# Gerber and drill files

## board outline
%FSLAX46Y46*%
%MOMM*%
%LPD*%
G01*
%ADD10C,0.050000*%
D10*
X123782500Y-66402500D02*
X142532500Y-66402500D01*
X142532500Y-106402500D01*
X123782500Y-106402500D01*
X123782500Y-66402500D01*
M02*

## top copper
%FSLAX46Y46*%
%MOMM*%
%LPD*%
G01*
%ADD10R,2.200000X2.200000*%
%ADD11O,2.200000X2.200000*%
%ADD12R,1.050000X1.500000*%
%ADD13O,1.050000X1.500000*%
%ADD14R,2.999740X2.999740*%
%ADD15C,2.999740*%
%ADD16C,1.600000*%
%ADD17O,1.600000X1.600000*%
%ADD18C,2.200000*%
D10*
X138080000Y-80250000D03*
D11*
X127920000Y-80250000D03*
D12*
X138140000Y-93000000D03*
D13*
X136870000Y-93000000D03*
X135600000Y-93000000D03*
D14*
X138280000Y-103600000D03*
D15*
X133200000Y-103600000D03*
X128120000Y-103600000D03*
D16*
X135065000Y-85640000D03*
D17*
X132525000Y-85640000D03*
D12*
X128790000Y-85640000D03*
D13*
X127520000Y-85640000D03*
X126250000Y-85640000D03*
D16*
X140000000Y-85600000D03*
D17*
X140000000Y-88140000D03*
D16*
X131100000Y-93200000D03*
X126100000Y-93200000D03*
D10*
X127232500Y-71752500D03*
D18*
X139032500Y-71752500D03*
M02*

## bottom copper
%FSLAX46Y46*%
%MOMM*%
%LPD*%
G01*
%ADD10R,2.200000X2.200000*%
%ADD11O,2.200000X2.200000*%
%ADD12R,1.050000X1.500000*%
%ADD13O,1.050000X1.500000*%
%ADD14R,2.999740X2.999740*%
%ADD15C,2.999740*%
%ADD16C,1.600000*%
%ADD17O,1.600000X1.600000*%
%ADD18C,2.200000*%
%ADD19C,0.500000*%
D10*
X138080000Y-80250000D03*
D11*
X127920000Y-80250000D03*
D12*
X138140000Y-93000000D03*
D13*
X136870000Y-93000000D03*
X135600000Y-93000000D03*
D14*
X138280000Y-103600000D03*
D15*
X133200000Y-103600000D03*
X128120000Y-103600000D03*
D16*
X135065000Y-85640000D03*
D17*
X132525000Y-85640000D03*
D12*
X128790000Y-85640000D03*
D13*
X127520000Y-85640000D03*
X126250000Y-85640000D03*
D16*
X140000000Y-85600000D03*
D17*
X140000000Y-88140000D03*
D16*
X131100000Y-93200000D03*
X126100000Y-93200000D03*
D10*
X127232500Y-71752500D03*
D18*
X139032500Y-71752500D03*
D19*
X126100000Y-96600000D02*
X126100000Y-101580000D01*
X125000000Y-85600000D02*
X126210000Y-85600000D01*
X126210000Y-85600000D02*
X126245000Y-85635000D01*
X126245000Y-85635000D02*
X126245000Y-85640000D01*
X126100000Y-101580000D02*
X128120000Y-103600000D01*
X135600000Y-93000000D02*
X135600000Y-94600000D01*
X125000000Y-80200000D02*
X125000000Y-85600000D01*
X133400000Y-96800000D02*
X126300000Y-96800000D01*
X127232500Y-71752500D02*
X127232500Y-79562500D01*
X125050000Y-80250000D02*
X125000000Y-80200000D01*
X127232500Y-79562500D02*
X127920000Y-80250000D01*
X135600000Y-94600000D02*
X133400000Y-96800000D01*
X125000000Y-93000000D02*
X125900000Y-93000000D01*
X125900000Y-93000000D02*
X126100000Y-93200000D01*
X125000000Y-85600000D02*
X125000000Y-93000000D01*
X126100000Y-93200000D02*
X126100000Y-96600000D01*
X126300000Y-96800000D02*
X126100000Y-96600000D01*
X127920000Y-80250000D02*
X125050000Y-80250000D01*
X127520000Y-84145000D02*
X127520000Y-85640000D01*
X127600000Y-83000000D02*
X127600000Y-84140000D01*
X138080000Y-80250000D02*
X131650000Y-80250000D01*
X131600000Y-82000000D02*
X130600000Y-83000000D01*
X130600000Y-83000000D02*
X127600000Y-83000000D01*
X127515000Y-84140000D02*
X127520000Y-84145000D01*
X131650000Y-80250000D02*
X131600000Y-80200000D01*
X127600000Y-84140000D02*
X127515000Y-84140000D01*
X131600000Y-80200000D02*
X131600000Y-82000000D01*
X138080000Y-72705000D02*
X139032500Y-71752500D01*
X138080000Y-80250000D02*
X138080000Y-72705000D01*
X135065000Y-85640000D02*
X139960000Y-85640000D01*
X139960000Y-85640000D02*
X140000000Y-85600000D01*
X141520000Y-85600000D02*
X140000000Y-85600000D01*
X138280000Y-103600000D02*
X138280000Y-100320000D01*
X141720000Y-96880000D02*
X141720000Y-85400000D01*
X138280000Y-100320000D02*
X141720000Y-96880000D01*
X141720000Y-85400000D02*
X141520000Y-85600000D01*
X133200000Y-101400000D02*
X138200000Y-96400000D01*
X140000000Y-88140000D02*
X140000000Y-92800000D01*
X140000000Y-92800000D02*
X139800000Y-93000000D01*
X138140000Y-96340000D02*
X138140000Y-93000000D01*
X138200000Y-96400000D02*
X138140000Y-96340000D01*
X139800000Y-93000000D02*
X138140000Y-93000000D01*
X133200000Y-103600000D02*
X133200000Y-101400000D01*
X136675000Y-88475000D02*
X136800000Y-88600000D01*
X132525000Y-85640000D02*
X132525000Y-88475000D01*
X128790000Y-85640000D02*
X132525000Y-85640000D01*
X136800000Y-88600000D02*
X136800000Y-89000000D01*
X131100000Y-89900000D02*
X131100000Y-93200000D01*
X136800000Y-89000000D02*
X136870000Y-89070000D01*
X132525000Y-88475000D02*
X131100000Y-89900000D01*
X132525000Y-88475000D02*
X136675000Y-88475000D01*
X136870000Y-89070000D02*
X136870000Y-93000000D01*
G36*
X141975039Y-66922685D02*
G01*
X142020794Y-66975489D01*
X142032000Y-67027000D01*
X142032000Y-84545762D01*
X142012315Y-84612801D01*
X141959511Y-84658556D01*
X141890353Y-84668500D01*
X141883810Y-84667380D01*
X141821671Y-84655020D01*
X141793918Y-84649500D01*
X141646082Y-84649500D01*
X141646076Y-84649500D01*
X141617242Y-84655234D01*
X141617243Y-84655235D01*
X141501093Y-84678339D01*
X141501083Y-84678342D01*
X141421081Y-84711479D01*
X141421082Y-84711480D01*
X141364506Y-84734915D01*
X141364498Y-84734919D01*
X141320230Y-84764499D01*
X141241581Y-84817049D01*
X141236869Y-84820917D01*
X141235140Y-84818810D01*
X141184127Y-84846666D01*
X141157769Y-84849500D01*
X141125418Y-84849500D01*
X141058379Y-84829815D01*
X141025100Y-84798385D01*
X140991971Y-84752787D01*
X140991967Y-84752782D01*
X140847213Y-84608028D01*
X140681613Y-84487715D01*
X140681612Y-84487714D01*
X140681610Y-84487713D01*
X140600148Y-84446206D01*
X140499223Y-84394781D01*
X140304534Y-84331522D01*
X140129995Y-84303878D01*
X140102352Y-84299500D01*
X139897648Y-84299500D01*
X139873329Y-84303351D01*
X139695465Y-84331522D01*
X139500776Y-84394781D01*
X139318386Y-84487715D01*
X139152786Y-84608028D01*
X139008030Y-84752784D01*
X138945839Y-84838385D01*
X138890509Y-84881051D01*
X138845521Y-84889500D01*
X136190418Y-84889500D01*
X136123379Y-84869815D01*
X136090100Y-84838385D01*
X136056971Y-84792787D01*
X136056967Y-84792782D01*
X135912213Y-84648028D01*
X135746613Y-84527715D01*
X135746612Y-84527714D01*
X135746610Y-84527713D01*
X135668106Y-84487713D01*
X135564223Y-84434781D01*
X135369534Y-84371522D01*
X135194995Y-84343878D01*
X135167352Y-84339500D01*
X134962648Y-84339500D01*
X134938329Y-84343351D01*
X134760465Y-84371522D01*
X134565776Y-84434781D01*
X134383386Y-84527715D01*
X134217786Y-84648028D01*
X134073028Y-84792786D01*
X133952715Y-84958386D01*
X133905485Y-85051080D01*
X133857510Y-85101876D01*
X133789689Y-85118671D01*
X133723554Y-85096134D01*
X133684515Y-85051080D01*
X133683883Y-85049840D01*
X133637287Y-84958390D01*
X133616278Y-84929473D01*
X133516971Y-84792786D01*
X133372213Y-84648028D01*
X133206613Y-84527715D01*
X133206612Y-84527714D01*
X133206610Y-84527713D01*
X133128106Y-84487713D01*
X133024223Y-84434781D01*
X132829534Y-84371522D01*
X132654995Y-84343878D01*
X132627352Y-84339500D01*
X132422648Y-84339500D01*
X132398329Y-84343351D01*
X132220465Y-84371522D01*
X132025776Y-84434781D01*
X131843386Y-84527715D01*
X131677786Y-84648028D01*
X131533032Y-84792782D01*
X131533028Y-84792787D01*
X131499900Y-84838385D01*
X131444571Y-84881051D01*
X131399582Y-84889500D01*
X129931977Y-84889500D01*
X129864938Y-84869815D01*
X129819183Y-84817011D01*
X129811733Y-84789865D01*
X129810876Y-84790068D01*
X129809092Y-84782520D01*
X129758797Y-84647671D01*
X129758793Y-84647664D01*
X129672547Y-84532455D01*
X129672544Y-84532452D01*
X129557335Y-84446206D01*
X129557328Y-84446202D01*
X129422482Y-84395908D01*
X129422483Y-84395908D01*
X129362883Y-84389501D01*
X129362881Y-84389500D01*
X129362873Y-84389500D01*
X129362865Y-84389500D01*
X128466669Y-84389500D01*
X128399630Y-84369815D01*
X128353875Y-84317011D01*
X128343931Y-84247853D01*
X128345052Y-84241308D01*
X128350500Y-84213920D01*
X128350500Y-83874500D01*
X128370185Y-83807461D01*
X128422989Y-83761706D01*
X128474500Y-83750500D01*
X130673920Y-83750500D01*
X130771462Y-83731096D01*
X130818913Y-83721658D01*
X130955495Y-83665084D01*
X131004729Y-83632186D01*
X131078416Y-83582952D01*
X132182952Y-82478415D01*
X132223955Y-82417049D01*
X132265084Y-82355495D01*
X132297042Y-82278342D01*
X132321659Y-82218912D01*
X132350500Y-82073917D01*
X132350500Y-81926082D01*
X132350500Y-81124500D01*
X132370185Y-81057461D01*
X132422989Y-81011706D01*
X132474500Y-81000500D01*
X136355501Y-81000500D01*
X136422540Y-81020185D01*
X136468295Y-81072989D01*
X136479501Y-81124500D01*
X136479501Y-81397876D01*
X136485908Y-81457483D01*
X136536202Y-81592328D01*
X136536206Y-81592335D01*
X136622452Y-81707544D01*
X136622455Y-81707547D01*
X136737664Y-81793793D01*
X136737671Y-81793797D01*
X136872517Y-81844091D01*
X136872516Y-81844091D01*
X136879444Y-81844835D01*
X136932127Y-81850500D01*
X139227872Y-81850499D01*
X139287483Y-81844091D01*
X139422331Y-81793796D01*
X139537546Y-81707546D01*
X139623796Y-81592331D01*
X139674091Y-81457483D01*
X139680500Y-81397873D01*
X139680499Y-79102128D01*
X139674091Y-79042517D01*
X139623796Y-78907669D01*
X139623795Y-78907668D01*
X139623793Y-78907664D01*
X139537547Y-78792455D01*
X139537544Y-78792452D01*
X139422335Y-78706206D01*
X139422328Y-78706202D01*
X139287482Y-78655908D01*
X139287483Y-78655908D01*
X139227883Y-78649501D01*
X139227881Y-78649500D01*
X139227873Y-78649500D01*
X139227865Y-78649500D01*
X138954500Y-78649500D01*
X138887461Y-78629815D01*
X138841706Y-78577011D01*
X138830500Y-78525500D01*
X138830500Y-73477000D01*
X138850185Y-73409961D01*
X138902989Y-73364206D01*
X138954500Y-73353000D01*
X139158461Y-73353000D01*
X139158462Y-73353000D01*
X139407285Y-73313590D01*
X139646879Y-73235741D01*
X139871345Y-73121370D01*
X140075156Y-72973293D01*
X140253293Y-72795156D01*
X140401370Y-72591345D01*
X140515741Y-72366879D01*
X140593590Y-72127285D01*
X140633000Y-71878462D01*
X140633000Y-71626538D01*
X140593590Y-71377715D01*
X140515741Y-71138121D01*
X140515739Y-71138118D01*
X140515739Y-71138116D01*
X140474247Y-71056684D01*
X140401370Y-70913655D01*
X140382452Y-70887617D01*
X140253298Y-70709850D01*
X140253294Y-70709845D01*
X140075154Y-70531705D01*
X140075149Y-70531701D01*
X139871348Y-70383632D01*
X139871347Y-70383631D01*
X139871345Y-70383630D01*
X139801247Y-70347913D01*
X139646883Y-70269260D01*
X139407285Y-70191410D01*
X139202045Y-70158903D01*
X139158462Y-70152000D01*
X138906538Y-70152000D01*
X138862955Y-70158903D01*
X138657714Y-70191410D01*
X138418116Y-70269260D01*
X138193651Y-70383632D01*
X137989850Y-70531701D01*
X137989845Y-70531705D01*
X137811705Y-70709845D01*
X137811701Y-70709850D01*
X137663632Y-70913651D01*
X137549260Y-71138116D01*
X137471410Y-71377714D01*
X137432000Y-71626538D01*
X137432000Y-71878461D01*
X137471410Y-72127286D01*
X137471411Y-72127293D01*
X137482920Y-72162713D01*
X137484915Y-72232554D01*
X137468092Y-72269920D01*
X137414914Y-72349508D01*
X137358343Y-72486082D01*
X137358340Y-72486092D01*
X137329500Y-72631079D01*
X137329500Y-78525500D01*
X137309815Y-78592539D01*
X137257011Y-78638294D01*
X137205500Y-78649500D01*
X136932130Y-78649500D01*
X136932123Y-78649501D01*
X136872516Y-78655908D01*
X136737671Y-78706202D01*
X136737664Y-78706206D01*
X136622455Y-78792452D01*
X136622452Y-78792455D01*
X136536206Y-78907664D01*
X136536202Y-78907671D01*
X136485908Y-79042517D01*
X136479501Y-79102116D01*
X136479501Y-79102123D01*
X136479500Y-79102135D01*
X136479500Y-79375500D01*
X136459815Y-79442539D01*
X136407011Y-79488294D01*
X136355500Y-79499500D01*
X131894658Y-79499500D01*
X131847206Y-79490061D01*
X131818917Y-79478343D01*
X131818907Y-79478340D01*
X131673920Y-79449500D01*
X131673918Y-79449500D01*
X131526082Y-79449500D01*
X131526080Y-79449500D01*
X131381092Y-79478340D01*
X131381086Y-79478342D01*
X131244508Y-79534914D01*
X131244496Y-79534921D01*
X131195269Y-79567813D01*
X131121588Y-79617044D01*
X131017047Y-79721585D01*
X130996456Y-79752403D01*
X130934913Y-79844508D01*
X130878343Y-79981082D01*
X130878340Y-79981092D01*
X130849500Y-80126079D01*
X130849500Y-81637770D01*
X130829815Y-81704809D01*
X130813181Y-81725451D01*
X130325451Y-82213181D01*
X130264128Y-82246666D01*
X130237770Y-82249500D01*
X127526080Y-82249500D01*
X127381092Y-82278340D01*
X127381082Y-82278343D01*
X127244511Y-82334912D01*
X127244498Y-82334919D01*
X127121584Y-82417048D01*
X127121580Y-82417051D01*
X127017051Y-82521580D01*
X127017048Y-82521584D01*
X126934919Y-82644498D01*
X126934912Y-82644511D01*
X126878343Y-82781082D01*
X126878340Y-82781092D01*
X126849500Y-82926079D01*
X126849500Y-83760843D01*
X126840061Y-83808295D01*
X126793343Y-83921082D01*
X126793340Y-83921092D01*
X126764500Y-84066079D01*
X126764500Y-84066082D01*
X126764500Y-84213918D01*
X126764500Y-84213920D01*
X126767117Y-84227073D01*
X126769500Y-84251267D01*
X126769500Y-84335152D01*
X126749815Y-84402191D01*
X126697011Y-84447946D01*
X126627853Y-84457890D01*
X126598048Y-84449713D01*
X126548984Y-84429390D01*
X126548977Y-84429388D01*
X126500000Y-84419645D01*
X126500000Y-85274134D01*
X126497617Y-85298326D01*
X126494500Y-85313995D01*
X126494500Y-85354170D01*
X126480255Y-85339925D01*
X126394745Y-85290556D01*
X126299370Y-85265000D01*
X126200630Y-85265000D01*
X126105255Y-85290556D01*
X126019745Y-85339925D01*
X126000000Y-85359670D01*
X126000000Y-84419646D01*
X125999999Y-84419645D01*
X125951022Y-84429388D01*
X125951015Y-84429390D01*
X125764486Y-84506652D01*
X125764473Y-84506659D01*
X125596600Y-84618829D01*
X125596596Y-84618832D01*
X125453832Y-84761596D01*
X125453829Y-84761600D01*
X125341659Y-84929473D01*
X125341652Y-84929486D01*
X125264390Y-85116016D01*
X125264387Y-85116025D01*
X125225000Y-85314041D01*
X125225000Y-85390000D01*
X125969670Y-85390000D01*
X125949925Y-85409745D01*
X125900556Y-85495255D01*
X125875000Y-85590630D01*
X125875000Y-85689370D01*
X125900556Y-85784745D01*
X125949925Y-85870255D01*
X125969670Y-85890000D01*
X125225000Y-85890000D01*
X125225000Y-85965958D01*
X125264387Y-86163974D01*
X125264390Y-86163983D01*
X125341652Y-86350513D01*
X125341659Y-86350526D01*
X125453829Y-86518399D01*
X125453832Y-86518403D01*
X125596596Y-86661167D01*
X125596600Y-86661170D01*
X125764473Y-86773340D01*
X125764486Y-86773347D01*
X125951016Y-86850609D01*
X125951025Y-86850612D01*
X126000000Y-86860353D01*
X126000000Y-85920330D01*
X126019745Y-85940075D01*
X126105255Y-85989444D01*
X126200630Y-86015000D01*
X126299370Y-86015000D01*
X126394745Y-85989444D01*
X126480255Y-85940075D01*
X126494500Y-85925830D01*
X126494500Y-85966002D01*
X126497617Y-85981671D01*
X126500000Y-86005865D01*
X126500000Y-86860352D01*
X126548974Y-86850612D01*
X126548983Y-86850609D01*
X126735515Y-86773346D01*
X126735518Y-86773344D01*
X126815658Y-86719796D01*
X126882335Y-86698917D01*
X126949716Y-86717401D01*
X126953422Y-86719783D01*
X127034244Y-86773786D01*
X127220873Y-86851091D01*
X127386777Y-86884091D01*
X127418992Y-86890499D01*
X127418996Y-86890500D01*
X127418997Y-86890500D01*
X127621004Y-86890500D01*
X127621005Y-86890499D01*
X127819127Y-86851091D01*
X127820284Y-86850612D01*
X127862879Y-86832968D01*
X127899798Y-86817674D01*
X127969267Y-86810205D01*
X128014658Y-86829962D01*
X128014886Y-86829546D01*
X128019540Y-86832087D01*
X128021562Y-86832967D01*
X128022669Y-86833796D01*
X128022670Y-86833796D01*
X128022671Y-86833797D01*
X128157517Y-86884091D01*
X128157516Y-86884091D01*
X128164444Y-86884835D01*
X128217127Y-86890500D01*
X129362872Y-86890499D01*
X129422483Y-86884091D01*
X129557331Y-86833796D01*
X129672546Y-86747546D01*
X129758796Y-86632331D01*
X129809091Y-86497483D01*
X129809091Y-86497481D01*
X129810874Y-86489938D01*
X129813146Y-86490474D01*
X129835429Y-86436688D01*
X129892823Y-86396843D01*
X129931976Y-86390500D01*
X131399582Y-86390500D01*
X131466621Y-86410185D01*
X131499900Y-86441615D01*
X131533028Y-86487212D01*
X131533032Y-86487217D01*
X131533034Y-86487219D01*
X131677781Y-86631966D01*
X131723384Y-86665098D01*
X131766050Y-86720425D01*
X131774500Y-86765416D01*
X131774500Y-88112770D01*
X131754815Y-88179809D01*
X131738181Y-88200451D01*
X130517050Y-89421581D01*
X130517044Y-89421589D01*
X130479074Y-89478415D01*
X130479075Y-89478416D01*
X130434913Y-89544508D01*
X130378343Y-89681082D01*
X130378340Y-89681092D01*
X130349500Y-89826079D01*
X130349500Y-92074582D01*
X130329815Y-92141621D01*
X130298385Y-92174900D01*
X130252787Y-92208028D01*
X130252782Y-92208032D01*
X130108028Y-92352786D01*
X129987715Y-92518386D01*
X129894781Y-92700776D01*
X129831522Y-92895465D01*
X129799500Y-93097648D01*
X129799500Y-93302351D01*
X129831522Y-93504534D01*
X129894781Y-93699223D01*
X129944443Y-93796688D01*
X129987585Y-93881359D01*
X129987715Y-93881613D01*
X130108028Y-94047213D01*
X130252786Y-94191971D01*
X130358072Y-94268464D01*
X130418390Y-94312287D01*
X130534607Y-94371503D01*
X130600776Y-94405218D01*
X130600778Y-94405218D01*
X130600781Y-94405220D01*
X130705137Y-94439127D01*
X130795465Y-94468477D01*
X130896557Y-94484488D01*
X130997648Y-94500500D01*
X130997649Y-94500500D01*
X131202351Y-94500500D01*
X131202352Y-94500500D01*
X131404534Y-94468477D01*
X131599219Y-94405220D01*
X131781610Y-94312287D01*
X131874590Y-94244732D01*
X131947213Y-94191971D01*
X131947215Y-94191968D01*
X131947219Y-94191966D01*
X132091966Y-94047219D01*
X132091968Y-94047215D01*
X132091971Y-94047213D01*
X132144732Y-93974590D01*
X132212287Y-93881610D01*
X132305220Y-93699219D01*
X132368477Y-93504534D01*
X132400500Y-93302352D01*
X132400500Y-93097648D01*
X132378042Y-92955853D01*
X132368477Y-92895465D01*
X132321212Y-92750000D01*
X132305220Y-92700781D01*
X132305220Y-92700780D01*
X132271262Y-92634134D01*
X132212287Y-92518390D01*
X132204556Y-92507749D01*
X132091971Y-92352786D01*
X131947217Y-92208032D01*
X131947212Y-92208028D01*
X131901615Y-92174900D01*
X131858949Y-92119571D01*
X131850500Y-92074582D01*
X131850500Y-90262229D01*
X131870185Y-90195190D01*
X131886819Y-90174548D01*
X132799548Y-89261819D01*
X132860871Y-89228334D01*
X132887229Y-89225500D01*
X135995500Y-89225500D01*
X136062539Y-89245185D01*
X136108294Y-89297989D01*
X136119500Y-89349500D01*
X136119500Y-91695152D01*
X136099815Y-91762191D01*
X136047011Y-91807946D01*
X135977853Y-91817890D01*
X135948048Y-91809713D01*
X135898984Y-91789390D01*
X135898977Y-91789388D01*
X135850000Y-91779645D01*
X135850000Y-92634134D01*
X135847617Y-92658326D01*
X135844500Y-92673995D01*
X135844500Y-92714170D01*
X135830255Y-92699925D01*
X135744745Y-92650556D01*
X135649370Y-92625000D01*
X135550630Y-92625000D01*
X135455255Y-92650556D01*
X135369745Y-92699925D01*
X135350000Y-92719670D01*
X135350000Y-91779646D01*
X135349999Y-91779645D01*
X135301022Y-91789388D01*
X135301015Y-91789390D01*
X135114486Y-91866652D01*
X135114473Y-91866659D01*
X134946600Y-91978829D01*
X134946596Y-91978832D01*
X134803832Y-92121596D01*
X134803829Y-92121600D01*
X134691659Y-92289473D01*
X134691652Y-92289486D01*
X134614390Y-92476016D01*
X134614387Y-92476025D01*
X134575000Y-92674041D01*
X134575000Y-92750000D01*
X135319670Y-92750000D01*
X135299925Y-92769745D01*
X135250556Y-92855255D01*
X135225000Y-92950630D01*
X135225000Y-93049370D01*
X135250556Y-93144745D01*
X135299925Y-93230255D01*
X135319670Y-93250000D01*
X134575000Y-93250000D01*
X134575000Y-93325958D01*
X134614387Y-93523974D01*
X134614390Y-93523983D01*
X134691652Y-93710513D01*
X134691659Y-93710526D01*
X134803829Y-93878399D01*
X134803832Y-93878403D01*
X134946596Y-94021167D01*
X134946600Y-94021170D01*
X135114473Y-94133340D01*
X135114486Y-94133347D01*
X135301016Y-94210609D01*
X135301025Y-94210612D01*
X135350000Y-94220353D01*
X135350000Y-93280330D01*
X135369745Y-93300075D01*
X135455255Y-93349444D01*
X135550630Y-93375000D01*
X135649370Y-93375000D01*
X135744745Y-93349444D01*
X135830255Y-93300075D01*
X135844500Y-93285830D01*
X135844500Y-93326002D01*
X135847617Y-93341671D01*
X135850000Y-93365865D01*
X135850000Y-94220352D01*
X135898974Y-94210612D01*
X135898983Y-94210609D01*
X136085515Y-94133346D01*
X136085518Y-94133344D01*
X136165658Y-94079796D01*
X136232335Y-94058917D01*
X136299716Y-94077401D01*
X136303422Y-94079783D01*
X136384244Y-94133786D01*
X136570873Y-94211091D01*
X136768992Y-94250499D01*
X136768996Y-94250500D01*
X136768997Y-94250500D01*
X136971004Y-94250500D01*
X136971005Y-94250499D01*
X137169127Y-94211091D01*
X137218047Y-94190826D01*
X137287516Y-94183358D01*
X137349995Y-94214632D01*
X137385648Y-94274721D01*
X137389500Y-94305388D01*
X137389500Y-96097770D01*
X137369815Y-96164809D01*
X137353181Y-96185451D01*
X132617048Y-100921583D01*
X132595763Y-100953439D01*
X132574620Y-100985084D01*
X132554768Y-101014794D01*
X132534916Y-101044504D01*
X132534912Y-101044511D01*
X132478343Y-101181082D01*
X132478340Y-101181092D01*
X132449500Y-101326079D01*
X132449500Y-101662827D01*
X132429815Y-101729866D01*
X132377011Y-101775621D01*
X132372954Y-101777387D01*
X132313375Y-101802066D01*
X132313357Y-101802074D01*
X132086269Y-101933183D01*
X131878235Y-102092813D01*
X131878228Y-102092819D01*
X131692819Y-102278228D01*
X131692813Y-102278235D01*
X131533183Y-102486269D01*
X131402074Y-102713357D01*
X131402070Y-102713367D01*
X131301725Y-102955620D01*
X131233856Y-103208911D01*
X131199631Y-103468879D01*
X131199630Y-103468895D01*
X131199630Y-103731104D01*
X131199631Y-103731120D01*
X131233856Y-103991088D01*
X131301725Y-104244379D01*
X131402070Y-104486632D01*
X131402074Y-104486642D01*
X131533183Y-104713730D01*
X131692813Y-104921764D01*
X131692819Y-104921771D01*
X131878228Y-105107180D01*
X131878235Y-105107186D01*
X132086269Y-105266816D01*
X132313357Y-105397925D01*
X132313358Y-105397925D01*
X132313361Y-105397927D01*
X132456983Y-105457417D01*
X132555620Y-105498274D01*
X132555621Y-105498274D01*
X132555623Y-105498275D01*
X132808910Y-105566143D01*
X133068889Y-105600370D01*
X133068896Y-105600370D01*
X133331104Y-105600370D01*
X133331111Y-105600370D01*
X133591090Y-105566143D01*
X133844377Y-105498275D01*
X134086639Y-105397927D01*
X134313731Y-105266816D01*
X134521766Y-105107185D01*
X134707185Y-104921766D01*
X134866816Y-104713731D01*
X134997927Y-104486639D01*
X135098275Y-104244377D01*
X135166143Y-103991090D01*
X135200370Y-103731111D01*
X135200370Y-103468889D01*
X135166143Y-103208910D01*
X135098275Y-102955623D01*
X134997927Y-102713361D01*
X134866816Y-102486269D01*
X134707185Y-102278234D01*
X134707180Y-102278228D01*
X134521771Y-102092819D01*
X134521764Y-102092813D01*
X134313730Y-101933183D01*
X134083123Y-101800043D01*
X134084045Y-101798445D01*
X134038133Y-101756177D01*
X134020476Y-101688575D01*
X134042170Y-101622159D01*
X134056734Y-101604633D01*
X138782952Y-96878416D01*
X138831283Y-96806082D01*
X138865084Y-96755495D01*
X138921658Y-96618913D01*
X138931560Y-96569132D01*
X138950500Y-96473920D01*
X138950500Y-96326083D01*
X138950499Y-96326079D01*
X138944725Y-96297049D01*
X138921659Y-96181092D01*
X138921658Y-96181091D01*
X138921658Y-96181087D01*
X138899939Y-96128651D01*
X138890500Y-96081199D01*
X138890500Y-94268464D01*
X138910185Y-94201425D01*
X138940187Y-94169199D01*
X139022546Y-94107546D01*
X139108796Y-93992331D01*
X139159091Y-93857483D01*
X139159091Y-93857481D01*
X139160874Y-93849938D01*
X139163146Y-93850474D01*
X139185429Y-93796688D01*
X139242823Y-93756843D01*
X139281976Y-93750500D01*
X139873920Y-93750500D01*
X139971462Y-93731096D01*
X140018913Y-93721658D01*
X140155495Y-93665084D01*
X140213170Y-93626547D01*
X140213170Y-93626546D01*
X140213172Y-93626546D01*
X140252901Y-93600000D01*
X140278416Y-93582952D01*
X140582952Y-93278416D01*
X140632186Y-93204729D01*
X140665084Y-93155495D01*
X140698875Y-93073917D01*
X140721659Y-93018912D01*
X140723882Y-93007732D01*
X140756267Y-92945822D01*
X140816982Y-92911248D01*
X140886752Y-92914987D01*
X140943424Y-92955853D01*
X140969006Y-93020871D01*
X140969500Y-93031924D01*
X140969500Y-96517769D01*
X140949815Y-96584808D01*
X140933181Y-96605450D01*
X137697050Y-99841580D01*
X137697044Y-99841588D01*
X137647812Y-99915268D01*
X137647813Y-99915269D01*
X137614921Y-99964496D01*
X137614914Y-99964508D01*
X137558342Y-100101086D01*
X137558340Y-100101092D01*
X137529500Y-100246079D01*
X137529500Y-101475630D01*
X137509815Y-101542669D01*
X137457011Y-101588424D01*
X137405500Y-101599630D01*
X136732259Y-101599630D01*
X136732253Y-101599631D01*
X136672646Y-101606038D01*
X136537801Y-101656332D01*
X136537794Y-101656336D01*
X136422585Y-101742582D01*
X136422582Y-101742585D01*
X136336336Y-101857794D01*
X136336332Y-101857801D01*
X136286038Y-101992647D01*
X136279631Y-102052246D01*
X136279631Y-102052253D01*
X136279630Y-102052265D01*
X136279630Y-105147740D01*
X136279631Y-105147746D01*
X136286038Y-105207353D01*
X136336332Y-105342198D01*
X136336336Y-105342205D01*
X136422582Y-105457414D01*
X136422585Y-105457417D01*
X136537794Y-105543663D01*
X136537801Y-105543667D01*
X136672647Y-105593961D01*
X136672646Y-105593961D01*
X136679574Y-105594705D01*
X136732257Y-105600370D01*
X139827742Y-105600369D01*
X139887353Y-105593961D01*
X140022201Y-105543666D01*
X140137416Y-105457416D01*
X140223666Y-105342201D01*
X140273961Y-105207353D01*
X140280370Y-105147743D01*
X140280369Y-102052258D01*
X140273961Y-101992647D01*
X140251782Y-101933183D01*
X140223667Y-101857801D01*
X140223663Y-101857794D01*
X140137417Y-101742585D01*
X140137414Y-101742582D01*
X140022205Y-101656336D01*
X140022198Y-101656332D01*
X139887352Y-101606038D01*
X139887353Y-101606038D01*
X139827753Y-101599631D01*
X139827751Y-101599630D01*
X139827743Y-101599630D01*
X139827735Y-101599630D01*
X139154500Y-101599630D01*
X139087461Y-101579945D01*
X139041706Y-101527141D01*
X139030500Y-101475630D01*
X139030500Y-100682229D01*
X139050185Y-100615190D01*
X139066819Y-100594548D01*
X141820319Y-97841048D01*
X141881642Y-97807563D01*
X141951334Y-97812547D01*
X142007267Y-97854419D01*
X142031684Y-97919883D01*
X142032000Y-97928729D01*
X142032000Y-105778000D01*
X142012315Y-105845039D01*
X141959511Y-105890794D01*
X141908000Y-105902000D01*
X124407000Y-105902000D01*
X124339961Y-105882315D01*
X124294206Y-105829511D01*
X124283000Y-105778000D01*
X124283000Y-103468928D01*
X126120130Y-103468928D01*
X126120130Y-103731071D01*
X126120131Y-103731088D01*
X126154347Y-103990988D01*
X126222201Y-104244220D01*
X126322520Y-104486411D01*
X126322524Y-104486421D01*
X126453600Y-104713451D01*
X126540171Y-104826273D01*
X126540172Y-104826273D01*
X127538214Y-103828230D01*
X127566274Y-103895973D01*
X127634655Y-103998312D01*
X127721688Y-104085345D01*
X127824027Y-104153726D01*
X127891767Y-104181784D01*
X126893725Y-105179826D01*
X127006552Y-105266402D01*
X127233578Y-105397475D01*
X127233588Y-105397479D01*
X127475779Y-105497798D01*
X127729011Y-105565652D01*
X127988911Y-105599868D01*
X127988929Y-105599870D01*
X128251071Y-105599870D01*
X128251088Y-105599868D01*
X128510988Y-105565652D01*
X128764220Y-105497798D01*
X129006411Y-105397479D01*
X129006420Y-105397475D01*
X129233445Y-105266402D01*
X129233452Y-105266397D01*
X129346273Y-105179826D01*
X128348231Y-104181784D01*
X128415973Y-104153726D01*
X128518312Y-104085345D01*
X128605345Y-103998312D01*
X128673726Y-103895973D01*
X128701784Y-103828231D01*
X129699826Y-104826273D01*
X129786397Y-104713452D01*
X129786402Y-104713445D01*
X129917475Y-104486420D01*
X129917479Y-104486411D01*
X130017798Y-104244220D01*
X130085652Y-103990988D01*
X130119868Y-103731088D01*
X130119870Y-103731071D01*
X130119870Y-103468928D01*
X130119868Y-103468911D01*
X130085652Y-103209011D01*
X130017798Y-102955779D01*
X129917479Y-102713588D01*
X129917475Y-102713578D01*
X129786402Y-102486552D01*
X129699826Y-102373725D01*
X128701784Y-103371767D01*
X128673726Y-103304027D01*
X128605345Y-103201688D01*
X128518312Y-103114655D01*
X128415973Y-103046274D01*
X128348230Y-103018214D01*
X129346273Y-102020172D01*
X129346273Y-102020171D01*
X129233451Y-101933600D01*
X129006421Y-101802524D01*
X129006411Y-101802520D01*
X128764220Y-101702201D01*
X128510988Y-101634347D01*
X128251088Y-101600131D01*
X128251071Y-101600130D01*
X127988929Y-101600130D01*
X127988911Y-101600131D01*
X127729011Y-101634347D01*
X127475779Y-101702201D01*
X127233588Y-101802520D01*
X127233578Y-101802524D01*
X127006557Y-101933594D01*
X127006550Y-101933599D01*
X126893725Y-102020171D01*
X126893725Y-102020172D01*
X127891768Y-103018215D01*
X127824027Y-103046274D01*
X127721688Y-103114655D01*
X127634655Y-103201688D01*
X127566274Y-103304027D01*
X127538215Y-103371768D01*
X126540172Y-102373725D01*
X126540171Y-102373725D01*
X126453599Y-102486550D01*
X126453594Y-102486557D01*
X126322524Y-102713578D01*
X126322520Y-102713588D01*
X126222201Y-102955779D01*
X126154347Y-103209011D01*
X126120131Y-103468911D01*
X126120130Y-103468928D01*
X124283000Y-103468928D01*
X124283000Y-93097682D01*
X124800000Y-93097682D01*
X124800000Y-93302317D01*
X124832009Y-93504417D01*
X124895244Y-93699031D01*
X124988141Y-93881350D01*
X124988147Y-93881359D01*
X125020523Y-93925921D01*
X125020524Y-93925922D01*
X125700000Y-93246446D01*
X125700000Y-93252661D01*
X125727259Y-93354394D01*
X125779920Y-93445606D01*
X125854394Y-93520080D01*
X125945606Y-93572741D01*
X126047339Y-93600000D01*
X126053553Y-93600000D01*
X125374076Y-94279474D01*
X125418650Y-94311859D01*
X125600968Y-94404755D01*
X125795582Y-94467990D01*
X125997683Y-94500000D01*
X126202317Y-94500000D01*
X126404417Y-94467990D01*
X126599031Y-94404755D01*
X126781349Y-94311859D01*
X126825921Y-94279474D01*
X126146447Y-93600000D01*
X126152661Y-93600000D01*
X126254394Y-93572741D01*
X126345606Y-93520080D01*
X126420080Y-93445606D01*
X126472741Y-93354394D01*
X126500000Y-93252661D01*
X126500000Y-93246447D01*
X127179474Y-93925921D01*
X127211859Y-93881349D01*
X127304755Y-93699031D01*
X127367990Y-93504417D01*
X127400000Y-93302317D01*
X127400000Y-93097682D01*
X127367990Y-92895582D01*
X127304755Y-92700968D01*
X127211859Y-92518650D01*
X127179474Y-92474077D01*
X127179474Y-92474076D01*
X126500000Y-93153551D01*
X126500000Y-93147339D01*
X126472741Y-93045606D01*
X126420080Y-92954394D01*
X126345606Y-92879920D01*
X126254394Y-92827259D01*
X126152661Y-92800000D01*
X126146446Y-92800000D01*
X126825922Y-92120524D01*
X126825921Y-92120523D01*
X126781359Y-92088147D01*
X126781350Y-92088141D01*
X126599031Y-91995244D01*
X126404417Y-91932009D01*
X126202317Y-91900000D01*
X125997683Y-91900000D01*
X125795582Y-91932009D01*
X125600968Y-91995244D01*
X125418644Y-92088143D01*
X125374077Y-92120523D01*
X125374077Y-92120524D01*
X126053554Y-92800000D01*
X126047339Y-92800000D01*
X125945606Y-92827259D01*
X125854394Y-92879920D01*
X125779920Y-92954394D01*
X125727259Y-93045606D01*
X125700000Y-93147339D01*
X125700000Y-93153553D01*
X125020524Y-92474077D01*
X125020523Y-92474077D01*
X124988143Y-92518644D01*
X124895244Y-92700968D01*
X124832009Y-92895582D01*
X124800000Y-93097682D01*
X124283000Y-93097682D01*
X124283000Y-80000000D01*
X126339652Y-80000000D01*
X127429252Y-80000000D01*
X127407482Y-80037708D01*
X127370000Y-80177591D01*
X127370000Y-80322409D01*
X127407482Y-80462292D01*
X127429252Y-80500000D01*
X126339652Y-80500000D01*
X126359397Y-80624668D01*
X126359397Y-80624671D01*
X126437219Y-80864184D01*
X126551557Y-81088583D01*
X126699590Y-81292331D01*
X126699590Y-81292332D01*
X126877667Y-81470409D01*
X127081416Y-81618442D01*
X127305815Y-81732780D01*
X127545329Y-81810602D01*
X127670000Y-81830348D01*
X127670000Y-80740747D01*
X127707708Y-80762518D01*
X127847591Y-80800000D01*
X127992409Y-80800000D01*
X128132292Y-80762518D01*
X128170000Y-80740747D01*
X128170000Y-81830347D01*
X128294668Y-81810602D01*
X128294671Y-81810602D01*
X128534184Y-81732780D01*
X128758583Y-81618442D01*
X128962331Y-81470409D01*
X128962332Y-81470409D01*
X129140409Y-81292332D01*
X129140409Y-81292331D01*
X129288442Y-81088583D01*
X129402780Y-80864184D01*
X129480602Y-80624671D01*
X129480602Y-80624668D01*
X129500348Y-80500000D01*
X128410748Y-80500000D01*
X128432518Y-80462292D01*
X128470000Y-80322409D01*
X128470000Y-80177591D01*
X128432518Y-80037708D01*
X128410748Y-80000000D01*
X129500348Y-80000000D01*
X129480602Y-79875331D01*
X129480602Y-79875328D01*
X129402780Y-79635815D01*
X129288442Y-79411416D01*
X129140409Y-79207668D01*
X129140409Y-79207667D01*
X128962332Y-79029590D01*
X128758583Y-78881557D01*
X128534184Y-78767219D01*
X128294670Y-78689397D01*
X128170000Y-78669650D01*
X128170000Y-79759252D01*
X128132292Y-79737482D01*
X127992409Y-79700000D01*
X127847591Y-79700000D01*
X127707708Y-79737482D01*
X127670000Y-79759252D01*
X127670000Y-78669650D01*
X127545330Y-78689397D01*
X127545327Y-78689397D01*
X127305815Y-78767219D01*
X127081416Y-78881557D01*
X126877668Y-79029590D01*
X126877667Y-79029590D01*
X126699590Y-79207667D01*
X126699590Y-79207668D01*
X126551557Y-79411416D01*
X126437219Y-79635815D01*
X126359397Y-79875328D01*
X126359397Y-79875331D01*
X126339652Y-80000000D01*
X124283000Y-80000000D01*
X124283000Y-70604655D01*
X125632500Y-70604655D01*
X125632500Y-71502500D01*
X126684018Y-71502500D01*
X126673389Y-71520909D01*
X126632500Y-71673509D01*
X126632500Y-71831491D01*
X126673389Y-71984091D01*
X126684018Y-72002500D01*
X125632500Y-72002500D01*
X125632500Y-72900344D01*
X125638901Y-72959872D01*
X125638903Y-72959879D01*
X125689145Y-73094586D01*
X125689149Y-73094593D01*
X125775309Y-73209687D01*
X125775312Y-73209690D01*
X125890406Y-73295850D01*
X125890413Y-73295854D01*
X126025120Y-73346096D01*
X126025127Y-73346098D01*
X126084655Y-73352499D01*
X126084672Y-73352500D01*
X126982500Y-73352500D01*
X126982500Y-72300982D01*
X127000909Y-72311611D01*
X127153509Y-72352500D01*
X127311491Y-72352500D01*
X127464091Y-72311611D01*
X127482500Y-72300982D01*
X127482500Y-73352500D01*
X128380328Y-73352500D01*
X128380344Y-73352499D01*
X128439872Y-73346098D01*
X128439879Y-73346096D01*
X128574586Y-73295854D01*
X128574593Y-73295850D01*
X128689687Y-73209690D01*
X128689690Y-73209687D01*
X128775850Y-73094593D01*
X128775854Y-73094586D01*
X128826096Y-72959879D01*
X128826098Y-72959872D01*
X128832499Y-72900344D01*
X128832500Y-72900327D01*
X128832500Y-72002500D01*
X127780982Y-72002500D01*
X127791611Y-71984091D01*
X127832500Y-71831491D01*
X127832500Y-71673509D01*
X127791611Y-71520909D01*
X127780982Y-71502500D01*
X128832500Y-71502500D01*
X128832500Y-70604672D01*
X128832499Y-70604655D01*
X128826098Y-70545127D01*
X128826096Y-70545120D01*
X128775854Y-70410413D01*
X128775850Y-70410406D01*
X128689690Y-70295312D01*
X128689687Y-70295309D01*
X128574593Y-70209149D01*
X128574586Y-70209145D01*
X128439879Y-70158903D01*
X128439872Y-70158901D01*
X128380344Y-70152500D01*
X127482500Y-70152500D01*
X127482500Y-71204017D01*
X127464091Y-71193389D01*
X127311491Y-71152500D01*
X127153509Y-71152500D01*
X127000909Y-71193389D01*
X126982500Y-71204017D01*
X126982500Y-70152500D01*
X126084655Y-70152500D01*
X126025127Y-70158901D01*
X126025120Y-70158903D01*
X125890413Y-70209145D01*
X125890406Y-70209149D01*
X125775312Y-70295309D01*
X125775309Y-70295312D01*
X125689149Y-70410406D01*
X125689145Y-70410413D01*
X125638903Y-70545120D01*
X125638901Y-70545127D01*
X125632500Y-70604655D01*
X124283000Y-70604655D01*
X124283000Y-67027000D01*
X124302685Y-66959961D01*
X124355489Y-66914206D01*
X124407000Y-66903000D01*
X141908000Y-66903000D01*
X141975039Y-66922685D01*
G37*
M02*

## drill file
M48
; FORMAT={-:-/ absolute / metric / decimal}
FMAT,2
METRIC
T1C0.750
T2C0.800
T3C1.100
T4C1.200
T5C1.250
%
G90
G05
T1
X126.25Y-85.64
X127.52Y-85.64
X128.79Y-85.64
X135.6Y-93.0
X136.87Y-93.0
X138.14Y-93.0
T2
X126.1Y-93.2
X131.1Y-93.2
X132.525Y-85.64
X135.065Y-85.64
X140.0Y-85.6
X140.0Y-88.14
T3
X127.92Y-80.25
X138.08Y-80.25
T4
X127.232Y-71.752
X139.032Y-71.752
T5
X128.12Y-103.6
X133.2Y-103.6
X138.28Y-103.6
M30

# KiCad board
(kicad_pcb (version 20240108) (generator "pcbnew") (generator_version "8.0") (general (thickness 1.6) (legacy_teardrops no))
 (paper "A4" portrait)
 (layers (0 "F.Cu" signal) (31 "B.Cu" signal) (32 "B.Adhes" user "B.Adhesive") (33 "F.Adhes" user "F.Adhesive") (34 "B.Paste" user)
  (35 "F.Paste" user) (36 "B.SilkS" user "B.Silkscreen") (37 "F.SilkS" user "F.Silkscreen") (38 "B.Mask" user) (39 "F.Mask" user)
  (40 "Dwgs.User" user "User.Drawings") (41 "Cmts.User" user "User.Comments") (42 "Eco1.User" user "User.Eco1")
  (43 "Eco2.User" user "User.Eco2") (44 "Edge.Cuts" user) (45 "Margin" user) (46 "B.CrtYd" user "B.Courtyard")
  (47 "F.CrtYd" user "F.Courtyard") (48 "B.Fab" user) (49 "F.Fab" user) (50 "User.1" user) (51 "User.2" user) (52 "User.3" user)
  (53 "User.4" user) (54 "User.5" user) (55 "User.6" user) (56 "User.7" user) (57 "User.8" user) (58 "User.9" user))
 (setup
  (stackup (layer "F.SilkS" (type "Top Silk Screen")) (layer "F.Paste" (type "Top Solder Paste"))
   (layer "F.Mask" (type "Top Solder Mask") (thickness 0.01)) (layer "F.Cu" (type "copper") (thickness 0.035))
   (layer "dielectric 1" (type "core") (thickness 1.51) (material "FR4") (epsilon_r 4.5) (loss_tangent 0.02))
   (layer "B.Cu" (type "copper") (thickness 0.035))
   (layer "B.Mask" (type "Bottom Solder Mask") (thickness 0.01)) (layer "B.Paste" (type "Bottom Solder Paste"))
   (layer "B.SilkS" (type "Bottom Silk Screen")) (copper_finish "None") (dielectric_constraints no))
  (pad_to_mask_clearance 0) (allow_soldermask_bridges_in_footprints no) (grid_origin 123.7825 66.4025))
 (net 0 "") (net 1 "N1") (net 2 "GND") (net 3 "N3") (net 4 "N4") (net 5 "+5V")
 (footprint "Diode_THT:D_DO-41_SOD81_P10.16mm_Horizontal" (layer "F.Cu") (at 138.08 80.25 180)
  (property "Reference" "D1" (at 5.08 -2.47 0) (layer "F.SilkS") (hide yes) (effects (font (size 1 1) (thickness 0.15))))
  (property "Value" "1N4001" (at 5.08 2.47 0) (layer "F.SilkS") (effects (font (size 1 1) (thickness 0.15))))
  (pad "1" thru_hole rect (at 0 0 180) (size 2.2 2.2) (drill 1.1) (layers "*.Cu" "*.Mask") (remove_unused_layers no) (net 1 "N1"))
  (pad "2" thru_hole oval (at 10.16 0 180) (size 2.2 2.2) (drill 1.1) (layers "*.Cu" "*.Mask") (remove_unused_layers no) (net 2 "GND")))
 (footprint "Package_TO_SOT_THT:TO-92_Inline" (layer "F.Cu") (at 138.14 93 180)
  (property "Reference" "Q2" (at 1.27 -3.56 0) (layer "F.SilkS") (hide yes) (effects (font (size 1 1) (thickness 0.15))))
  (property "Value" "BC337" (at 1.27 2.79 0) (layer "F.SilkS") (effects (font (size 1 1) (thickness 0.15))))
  (pad "1" thru_hole rect (at 0 0 180) (size 1.05 1.5) (drill 0.75) (layers "*.Cu" "*.Mask") (remove_unused_layers no) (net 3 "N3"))
  (pad "2" thru_hole oval (at 1.27 0 180) (size 1.05 1.5) (drill 0.75) (layers "*.Cu" "*.Mask") (remove_unused_layers no) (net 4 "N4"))
  (pad "3" thru_hole oval (at 2.54 0 180) (size 1.05 1.5) (drill 0.75) (layers "*.Cu" "*.Mask") (remove_unused_layers no) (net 2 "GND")))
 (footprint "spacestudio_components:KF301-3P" (layer "F.Cu") (at 133.2 103.6 180)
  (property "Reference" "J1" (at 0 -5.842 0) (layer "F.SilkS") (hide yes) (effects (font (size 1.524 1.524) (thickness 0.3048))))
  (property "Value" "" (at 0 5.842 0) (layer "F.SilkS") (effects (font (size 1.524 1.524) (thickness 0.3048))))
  (pad "1" thru_hole rect (at -5.08 0 180) (size 2.99974 2.99974) (drill 1.24968) (layers "*.Cu" "*.Mask" "F.SilkS")
   (remove_unused_layers no) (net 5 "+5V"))
  (pad "2" thru_hole circle (at 0 0 180) (size 2.99974 2.99974) (drill 1.24968) (layers "*.Cu" "*.Mask" "F.SilkS") (remove_unused_layers no)
   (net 3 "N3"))
  (pad "3" thru_hole circle (at 5.08 0 180) (size 2.99974 2.99974) (drill 1.24968) (layers "*.Cu" "*.Mask" "F.SilkS")
   (remove_unused_layers no) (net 2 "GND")))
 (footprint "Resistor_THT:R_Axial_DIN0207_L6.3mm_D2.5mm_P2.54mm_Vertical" (layer "F.Cu") (at 135.065 85.64 180)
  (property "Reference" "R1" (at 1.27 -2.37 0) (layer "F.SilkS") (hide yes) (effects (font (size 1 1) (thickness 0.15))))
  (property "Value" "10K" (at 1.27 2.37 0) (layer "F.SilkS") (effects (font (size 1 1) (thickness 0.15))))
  (pad "1" thru_hole circle (at 0 0 180) (size 1.6 1.6) (drill 0.8) (layers "*.Cu" "*.Mask") (remove_unused_layers no) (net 5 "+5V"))
  (pad "2" thru_hole oval (at 2.54 0 180) (size 1.6 1.6) (drill 0.8) (layers "*.Cu" "*.Mask") (remove_unused_layers no) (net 4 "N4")))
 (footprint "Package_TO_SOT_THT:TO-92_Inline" (layer "F.Cu") (at 128.79 85.64 180)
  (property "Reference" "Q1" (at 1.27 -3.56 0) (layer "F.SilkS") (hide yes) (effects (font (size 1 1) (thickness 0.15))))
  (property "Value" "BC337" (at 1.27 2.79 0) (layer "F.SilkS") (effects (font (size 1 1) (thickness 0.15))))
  (pad "1" thru_hole rect (at 0 0 180) (size 1.05 1.5) (drill 0.75) (layers "*.Cu" "*.Mask") (remove_unused_layers no) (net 4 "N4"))
  (pad "2" thru_hole oval (at 1.27 0 180) (size 1.05 1.5) (drill 0.75) (layers "*.Cu" "*.Mask") (remove_unused_layers no) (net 1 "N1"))
  (pad "3" thru_hole oval (at 2.54 0 180) (size 1.05 1.5) (drill 0.75) (layers "*.Cu" "*.Mask") (remove_unused_layers no) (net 2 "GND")))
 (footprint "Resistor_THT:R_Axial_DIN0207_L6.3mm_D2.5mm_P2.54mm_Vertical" (layer "F.Cu") (at 140 85.6 -90)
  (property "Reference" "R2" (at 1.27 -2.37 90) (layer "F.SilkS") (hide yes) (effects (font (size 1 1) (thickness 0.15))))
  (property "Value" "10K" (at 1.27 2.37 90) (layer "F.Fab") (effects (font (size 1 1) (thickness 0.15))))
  (pad "1" thru_hole circle (at 0 0 270) (size 1.6 1.6) (drill 0.8) (layers "*.Cu" "*.Mask") (remove_unused_layers no) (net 5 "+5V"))
  (pad "2" thru_hole oval (at 2.54 0 270) (size 1.6 1.6) (drill 0.8) (layers "*.Cu" "*.Mask") (remove_unused_layers no) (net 3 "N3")))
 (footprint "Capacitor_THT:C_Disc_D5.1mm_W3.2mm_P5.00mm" (layer "F.Cu") (at 131.1 93.2 180)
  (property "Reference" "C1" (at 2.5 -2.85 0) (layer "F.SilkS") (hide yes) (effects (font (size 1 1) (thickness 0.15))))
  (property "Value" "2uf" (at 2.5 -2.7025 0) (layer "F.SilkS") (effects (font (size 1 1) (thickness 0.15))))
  (pad "1" thru_hole circle (at 0 0 180) (size 1.6 1.6) (drill 0.8) (layers "*.Cu" "*.Mask") (remove_unused_layers no) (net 4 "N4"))
  (pad "2" thru_hole circle (at 5 0 180) (size 1.6 1.6) (drill 0.8) (layers "*.Cu" "*.Mask") (remove_unused_layers no) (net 2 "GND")))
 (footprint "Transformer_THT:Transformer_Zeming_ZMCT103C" (layer "F.Cu") (at 127.2325 71.7525)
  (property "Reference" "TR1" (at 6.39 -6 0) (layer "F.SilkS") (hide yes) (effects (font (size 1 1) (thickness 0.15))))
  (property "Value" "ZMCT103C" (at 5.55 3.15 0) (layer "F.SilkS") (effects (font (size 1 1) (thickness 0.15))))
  (pad "1" thru_hole rect (at 0 0) (size 2.2 2.2) (drill 1.2) (layers "*.Cu" "*.Mask") (remove_unused_layers no) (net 2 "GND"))
  (pad "2" thru_hole circle (at 11.8 0) (size 2.2 2.2) (drill 1.2) (layers "*.Cu" "*.Mask") (remove_unused_layers no) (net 1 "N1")))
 (gr_rect (start 123.7825 66.4025) (end 142.5325 106.4025) (stroke (width 0.05) (type default)) (fill none) (layer "Edge.Cuts"))
 (segment (start 126.1 96.6) (end 126.1 101.58) (width 0.5) (layer "B.Cu") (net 2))
 (segment (start 125 85.6) (end 126.21 85.6) (width 0.5) (layer "B.Cu") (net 2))
 (segment (start 126.21 85.6) (end 126.245 85.635) (width 0.5) (layer "B.Cu") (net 2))
 (segment (start 126.245 85.635) (end 126.245 85.64) (width 0.5) (layer "B.Cu") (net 2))
 (segment (start 126.1 101.58) (end 128.12 103.6) (width 0.5) (layer "B.Cu") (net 2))
 (segment (start 135.6 93) (end 135.6 94.6) (width 0.5) (layer "B.Cu") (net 2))
 (segment (start 125 80.2) (end 125 85.6) (width 0.5) (layer "B.Cu") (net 2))
 (segment (start 133.4 96.8) (end 126.3 96.8) (width 0.5) (layer "B.Cu") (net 2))
 (segment (start 127.2325 71.7525) (end 127.2325 79.5625) (width 0.5) (layer "B.Cu") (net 2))
 (segment (start 125.05 80.25) (end 125 80.2) (width 0.5) (layer "B.Cu") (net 2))
 (segment (start 127.2325 79.5625) (end 127.92 80.25) (width 0.5) (layer "B.Cu") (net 2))
 (segment (start 135.6 94.6) (end 133.4 96.8) (width 0.5) (layer "B.Cu") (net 2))
 (segment (start 125 93) (end 125.9 93) (width 0.5) (layer "B.Cu") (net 2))
 (segment (start 125.9 93) (end 126.1 93.2) (width 0.5) (layer "B.Cu") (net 2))
 (segment (start 125 85.6) (end 125 93) (width 0.5) (layer "B.Cu") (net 2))
 (segment (start 126.1 93.2) (end 126.1 96.6) (width 0.5) (layer "B.Cu") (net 2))
 (segment (start 126.3 96.8) (end 126.1 96.6) (width 0.5) (layer "B.Cu") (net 2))
 (segment (start 127.92 80.25) (end 125.05 80.25) (width 0.5) (layer "B.Cu") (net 2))
 (segment (start 127.52 84.145) (end 127.52 85.64) (width 0.5) (layer "B.Cu") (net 1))
 (segment (start 127.6 83) (end 127.6 84.14) (width 0.5) (layer "B.Cu") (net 1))
 (segment (start 138.08 80.25) (end 131.65 80.25) (width 0.5) (layer "B.Cu") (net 1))
 (segment (start 131.6 82) (end 130.6 83) (width 0.5) (layer "B.Cu") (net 1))
 (segment (start 130.6 83) (end 127.6 83) (width 0.5) (layer "B.Cu") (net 1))
 (segment (start 127.515 84.14) (end 127.52 84.145) (width 0.5) (layer "B.Cu") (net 1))
 (segment (start 131.65 80.25) (end 131.6 80.2) (width 0.5) (layer "B.Cu") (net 1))
 (segment (start 127.6 84.14) (end 127.515 84.14) (width 0.5) (layer "B.Cu") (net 1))
 (segment (start 131.6 80.2) (end 131.6 82) (width 0.5) (layer "B.Cu") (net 1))
 (segment (start 138.08 72.705) (end 139.0325 71.7525) (width 0.5) (layer "B.Cu") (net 1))
 (segment (start 138.08 80.25) (end 138.08 72.705) (width 0.5) (layer "B.Cu") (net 1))
 (segment (start 135.065 85.64) (end 139.96 85.64) (width 0.5) (layer "B.Cu") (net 5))
 (segment (start 139.96 85.64) (end 140 85.6) (width 0.5) (layer "B.Cu") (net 5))
 (segment (start 141.52 85.6) (end 140 85.6) (width 0.5) (layer "B.Cu") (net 5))
 (segment (start 138.28 103.6) (end 138.28 100.32) (width 0.5) (layer "B.Cu") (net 5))
 (segment (start 141.72 96.88) (end 141.72 85.4) (width 0.5) (layer "B.Cu") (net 5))
 (segment (start 138.28 100.32) (end 141.72 96.88) (width 0.5) (layer "B.Cu") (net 5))
 (segment (start 141.72 85.4) (end 141.52 85.6) (width 0.5) (layer "B.Cu") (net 5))
 (segment (start 133.2 101.4) (end 138.2 96.4) (width 0.5) (layer "B.Cu") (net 3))
 (segment (start 140 88.14) (end 140 92.8) (width 0.5) (layer "B.Cu") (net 3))
 (segment (start 140 92.8) (end 139.8 93) (width 0.5) (layer "B.Cu") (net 3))
 (segment (start 138.14 96.34) (end 138.14 93) (width 0.5) (layer "B.Cu") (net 3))
 (segment (start 138.2 96.4) (end 138.14 96.34) (width 0.5) (layer "B.Cu") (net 3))
 (segment (start 139.8 93) (end 138.14 93) (width 0.5) (layer "B.Cu") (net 3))
 (segment (start 133.2 103.6) (end 133.2 101.4) (width 0.5) (layer "B.Cu") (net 3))
 (segment (start 136.675 88.475) (end 136.8 88.6) (width 0.5) (layer "B.Cu") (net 4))
 (segment (start 132.525 85.64) (end 132.525 88.475) (width 0.5) (layer "B.Cu") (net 4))
 (segment (start 128.79 85.64) (end 132.525 85.64) (width 0.5) (layer "B.Cu") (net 4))
 (segment (start 136.8 88.6) (end 136.8 89) (width 0.5) (layer "B.Cu") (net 4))
 (segment (start 131.1 89.9) (end 131.1 93.2) (width 0.5) (layer "B.Cu") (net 4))
 (segment (start 136.8 89) (end 136.87 89.07) (width 0.5) (layer "B.Cu") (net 4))
 (segment (start 132.525 88.475) (end 131.1 89.9) (width 0.5) (layer "B.Cu") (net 4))
 (segment (start 132.525 88.475) (end 136.675 88.475) (width 0.5) (layer "B.Cu") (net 4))
 (segment (start 136.87 89.07) (end 136.87 93) (width 0.5) (layer "B.Cu") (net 4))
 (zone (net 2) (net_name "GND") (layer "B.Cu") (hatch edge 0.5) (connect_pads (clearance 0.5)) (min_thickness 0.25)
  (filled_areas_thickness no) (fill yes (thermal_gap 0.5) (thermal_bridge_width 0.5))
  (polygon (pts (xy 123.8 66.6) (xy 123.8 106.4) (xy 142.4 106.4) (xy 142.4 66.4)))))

